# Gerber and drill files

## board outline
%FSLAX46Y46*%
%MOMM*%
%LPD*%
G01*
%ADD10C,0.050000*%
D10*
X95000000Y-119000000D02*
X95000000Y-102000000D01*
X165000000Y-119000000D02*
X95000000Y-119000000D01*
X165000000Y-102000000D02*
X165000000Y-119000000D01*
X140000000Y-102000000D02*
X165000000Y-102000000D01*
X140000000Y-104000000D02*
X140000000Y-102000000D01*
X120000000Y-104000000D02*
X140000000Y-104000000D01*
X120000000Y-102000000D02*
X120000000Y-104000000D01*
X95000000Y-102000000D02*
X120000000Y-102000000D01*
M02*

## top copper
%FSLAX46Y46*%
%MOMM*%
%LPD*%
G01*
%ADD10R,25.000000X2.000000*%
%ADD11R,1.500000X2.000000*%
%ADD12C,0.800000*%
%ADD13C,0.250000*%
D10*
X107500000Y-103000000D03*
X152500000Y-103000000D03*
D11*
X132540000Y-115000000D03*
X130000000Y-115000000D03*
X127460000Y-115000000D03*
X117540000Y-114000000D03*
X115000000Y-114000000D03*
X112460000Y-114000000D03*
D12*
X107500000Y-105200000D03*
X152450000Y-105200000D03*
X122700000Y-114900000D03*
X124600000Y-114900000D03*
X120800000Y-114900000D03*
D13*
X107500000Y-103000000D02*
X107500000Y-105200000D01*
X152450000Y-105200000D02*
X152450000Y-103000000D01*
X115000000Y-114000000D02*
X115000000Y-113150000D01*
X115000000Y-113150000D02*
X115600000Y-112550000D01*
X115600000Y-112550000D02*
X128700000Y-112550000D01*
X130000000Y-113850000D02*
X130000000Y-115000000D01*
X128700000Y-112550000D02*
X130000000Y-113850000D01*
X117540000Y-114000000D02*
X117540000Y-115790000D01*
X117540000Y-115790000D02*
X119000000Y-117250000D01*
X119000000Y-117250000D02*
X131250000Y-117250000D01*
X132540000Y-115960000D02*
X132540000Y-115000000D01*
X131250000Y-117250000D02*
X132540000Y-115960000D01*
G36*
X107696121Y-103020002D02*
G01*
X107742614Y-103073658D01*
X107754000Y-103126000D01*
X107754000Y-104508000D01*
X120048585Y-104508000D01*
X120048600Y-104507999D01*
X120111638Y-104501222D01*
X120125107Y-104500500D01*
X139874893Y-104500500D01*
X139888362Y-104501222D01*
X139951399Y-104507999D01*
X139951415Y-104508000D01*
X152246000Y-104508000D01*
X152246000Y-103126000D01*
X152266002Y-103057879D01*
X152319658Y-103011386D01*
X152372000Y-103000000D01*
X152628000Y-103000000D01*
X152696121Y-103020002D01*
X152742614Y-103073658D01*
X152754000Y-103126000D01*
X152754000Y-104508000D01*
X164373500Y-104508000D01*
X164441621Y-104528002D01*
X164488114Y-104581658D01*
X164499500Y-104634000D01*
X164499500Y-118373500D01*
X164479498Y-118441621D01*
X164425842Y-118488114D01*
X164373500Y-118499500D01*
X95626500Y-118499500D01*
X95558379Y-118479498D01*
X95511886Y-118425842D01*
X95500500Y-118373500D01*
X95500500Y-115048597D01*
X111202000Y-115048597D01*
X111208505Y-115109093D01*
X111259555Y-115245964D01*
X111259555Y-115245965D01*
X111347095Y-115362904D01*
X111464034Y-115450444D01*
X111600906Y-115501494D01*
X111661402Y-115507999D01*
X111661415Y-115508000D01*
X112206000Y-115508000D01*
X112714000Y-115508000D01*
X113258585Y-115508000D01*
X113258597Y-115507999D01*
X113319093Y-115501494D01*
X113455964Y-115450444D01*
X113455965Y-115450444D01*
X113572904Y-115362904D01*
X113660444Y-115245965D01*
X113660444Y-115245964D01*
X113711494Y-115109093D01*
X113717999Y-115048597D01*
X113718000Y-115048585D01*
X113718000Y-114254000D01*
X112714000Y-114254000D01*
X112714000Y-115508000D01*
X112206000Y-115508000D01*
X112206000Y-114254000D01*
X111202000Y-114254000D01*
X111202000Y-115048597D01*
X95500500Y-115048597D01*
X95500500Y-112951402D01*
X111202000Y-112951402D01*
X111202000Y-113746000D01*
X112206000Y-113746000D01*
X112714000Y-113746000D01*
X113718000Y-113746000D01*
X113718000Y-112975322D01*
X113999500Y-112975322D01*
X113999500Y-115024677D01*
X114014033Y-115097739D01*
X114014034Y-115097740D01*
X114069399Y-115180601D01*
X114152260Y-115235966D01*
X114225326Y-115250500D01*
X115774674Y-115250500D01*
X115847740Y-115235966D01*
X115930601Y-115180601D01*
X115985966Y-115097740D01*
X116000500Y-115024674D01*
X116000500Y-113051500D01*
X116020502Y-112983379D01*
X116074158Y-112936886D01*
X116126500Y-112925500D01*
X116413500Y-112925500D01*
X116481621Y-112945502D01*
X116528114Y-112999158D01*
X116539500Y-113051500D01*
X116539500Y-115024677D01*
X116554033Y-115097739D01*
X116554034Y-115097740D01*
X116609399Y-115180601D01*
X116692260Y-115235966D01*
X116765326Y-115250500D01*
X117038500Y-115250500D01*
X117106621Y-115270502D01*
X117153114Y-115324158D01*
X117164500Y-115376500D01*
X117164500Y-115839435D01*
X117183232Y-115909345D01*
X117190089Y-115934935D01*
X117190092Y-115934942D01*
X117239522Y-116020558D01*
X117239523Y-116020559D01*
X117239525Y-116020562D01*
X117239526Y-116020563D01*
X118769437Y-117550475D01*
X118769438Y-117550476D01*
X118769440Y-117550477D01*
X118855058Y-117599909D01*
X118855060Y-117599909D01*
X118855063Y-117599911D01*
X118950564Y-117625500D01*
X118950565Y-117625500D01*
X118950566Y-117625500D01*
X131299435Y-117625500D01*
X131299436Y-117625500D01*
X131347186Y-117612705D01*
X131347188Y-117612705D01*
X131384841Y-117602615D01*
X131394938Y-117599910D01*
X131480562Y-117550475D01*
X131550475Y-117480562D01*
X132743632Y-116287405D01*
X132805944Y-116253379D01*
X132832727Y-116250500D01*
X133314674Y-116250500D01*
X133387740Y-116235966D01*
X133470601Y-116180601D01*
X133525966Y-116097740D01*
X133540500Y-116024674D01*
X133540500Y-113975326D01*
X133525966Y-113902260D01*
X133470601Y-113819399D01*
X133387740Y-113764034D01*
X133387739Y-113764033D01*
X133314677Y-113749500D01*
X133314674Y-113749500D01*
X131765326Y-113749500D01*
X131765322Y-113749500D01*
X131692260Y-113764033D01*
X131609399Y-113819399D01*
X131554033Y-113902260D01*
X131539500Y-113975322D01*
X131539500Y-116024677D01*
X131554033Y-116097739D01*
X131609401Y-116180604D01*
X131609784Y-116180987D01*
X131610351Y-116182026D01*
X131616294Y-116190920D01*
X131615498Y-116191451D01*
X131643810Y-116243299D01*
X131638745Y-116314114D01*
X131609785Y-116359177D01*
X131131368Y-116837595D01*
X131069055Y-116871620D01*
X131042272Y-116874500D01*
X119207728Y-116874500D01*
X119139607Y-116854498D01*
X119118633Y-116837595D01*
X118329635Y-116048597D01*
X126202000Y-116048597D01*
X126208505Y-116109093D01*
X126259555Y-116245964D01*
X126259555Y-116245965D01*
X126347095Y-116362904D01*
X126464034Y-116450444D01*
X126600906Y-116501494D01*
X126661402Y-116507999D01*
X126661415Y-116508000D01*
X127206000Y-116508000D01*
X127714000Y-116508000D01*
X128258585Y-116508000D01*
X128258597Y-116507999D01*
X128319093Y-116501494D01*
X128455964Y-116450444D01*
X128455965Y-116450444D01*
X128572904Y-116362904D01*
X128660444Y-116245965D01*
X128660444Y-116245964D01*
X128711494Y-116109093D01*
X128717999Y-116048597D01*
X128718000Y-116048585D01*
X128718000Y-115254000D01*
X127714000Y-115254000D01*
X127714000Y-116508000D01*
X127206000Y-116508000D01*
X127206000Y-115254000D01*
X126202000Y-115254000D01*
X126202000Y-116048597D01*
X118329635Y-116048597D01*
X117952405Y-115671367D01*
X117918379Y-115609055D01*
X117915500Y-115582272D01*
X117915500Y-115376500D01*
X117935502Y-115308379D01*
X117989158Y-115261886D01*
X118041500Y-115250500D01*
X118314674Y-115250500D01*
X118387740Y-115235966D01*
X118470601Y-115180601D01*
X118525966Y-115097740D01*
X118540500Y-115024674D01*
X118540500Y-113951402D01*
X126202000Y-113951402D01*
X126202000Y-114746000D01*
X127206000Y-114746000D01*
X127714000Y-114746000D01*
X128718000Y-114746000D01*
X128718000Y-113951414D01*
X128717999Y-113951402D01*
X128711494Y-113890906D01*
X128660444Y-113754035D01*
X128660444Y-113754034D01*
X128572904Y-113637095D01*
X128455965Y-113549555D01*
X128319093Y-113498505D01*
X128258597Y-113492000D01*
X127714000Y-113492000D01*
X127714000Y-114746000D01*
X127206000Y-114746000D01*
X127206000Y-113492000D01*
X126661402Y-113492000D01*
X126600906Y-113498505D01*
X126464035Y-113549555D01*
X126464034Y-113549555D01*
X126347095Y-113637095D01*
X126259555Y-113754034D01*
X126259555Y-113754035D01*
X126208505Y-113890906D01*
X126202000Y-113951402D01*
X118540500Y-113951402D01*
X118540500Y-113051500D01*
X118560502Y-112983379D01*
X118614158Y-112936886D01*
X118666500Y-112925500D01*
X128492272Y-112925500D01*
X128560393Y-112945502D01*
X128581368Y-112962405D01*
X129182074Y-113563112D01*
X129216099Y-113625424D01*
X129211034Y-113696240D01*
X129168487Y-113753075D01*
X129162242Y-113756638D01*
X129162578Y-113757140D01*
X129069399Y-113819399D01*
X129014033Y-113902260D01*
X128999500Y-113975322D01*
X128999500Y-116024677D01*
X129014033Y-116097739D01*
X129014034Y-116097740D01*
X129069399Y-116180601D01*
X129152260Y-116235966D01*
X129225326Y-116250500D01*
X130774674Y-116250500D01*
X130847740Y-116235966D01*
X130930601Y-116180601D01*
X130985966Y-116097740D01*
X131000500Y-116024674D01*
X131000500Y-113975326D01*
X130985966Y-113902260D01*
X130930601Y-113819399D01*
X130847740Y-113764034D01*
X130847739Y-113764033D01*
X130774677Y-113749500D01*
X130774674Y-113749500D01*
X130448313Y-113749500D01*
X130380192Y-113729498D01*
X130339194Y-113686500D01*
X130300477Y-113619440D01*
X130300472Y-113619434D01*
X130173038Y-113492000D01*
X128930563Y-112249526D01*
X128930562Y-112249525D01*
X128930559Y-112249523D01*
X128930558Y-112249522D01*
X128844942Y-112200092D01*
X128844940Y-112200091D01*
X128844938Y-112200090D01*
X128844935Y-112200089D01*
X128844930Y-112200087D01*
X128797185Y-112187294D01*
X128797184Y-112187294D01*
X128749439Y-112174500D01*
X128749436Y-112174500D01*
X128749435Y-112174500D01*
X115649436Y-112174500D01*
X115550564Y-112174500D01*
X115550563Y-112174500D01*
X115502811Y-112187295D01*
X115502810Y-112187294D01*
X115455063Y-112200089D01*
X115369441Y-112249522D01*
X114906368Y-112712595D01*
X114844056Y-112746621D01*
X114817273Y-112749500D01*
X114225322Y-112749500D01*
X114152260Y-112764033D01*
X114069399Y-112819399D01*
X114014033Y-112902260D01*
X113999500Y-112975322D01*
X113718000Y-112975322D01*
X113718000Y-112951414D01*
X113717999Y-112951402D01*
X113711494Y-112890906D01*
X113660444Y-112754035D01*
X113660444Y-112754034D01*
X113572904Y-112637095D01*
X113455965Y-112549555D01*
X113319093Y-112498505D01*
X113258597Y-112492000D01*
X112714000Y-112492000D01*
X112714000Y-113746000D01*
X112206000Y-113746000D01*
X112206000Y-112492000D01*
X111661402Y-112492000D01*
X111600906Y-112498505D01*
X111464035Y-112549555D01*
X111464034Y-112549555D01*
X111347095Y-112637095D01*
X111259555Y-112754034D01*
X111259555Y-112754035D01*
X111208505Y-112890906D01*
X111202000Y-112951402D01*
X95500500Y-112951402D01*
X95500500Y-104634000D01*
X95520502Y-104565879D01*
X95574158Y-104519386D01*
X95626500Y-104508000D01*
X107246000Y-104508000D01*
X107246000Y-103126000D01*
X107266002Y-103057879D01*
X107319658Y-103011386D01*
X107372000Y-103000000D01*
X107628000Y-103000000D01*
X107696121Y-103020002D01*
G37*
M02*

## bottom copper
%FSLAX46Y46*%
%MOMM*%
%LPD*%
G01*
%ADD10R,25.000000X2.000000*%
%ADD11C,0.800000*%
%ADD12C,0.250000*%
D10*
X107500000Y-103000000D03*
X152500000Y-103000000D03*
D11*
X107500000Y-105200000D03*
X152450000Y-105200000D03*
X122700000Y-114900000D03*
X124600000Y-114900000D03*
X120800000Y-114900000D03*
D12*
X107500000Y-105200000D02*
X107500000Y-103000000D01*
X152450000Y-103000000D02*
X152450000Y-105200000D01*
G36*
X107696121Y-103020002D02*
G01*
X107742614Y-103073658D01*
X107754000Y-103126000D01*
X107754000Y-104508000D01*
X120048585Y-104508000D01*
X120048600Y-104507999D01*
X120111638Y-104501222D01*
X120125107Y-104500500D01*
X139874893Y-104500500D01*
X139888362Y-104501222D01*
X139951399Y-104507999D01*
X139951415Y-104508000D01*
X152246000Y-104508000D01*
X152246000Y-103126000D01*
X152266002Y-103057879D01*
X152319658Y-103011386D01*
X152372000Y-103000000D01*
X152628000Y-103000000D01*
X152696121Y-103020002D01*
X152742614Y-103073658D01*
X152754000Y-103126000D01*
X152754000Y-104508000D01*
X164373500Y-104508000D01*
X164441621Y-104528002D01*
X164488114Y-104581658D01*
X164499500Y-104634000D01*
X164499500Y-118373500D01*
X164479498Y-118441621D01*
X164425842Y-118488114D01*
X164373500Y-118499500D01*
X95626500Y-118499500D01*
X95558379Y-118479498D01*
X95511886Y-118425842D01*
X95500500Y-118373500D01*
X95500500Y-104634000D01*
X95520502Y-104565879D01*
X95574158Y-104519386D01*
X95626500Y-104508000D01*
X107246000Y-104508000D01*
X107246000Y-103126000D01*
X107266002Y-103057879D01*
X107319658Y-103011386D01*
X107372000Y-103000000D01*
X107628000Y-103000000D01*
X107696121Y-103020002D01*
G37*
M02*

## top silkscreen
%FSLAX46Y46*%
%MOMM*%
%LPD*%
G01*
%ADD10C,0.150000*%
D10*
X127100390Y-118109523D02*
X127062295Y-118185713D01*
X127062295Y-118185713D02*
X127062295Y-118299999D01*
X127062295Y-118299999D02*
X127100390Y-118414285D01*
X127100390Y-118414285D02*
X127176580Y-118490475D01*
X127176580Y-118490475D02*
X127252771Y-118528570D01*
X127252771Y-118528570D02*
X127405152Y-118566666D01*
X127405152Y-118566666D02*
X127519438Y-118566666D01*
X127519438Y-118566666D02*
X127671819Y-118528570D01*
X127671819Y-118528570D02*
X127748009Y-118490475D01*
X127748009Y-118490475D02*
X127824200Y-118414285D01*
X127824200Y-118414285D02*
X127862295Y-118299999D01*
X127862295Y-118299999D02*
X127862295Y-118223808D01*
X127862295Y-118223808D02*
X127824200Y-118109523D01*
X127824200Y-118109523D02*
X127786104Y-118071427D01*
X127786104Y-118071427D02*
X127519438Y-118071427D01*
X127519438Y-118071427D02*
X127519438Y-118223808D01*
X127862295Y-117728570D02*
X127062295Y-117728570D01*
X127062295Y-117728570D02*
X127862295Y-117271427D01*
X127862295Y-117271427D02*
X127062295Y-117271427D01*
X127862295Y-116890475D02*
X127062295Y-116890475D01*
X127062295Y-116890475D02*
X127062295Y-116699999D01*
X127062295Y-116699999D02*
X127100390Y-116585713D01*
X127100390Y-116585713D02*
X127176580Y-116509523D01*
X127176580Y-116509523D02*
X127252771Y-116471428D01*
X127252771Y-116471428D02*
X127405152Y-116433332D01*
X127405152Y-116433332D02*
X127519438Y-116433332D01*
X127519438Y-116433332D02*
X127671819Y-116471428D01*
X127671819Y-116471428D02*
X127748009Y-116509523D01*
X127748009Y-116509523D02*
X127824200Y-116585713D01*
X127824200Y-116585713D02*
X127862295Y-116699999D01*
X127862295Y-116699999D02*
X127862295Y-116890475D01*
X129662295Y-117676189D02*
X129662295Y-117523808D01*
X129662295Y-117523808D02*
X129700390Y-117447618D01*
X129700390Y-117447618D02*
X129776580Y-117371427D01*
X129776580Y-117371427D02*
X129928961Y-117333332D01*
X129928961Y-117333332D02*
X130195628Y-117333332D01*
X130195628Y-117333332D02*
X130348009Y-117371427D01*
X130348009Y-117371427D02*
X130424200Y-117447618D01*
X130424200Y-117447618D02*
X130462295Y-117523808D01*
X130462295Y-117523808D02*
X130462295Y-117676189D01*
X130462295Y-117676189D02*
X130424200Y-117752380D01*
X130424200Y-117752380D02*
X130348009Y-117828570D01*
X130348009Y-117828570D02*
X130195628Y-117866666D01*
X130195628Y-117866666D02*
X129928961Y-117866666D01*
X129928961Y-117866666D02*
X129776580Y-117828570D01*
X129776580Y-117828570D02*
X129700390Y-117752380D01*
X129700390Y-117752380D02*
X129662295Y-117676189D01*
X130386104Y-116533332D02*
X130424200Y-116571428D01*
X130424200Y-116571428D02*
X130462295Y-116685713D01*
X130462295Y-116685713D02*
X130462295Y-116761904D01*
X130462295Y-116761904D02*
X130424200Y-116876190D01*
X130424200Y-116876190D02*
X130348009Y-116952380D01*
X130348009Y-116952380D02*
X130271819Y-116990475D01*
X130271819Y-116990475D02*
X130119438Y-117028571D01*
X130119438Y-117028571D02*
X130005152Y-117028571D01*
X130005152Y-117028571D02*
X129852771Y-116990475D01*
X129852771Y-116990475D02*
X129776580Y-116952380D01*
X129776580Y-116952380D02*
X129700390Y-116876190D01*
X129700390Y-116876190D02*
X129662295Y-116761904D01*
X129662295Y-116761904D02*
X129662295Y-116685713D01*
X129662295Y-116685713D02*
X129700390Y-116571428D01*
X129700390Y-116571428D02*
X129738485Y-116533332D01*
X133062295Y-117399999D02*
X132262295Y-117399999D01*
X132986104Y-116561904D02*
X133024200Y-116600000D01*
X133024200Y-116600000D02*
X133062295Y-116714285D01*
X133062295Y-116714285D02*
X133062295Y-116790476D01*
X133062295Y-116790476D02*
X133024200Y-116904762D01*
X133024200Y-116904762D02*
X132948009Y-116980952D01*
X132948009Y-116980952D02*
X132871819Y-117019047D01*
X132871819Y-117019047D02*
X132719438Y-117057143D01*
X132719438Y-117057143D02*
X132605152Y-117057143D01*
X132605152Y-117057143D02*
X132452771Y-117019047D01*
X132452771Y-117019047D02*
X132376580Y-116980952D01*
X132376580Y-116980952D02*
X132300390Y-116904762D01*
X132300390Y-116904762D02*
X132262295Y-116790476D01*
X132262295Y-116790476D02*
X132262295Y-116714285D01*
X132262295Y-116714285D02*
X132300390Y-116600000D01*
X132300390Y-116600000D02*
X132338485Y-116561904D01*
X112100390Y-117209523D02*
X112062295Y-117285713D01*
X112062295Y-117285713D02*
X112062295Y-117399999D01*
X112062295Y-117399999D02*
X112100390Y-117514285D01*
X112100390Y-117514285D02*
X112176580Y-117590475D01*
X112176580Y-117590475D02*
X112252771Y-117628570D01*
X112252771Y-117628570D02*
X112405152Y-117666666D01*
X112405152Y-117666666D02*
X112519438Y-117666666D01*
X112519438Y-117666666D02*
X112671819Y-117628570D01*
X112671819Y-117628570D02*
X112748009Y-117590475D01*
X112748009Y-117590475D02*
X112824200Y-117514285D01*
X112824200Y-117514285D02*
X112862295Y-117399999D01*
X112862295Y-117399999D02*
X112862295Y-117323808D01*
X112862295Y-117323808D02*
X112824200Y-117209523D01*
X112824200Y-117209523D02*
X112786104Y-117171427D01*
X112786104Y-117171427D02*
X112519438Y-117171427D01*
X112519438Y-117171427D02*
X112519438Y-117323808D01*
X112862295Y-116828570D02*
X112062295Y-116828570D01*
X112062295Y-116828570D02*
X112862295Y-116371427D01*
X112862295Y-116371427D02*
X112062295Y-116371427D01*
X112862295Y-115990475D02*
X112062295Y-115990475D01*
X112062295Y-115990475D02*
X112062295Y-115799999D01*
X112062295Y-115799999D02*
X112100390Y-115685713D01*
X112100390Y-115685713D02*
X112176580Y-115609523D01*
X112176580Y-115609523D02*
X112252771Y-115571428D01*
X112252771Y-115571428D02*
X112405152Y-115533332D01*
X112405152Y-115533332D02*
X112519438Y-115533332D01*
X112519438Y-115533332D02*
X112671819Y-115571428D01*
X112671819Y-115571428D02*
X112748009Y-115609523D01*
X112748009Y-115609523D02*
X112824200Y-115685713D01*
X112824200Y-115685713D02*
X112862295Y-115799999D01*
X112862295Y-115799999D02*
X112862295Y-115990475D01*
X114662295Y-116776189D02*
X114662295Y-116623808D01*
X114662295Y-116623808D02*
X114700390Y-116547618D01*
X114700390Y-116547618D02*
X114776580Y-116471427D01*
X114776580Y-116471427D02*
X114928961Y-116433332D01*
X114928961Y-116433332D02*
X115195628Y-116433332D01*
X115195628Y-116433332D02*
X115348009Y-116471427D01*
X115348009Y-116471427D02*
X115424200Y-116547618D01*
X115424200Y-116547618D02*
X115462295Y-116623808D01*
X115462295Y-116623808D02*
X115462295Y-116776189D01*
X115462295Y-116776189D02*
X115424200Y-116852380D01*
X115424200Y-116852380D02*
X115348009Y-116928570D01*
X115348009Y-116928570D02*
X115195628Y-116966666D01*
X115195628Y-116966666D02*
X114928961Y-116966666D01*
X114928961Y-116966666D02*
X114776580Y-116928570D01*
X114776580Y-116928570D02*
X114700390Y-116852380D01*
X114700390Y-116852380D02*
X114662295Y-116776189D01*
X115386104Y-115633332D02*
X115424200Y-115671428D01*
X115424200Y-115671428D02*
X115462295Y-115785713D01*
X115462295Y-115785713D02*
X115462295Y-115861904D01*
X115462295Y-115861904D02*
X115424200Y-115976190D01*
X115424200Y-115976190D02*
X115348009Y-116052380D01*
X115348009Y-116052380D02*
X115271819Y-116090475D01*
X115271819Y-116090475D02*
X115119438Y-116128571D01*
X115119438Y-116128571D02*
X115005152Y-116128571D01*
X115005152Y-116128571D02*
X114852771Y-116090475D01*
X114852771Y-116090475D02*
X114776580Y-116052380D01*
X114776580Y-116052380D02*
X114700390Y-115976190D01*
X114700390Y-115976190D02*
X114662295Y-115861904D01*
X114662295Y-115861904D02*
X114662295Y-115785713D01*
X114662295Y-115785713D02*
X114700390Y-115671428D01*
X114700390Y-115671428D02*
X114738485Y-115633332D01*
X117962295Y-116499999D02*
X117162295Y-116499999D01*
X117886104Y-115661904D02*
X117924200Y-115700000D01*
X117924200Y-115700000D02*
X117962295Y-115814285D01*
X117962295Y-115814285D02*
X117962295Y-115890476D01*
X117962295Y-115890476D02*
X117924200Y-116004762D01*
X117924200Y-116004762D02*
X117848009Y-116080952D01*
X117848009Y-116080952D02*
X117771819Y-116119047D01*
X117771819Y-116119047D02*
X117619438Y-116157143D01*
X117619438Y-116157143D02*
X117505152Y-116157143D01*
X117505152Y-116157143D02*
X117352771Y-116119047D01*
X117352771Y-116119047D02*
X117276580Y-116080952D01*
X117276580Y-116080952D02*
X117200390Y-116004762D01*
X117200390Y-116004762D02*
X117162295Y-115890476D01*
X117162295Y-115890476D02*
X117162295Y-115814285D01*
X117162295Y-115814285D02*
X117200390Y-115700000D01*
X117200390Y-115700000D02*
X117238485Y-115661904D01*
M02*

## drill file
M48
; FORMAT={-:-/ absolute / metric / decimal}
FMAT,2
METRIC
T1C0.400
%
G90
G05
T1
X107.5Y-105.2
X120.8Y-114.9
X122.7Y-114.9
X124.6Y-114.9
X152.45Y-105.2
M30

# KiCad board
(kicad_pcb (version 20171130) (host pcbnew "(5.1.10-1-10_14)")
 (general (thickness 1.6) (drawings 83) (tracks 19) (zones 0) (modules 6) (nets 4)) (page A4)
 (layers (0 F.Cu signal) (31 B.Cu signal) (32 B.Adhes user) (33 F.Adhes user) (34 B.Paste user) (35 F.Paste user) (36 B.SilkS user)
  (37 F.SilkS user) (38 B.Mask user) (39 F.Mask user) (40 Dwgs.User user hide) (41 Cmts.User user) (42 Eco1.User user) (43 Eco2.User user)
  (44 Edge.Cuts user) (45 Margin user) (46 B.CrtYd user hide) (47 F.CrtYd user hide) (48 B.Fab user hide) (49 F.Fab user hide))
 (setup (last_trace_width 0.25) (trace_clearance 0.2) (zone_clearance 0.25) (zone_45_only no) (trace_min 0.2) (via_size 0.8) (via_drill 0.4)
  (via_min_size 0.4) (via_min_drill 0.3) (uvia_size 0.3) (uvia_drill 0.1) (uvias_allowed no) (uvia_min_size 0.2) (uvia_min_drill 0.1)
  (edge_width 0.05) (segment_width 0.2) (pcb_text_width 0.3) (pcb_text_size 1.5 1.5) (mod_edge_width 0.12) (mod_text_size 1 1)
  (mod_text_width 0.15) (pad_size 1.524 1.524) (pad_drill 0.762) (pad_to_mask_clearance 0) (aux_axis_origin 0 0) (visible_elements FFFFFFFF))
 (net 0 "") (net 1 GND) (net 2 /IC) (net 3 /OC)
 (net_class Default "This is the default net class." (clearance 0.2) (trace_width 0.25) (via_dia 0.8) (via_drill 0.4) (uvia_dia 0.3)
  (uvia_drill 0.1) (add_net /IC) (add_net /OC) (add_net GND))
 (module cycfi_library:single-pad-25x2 (layer F.Cu) (at 107.5 103)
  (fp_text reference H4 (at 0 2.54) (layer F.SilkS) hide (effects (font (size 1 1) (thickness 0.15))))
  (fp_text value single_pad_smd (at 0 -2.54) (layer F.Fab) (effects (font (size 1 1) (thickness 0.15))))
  (pad 1 smd rect (at 0 0) (size 25 2) (layers F.Cu F.Paste F.Mask) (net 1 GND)))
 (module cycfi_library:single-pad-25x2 (layer B.Cu) (at 107.5 103)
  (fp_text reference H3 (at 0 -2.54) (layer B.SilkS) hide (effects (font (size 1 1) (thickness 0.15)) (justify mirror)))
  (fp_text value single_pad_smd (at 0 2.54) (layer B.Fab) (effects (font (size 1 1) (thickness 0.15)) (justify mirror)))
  (pad 1 smd rect (at 0 0) (size 25 2) (layers B.Cu B.Paste B.Mask) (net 1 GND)))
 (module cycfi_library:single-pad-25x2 (layer F.Cu) (at 152.5 103)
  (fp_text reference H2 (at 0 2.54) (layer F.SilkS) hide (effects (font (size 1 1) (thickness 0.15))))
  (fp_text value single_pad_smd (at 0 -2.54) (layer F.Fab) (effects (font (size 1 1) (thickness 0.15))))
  (pad 1 smd rect (at 0 0) (size 25 2) (layers F.Cu F.Paste F.Mask) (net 1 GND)))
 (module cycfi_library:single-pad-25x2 (layer B.Cu) (at 152.5 103)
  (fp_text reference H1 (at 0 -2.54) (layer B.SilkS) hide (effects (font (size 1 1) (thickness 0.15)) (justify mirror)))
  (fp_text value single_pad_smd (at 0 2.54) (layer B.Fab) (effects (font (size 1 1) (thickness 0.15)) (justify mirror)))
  (pad 1 smd rect (at 0 0) (size 25 2) (layers B.Cu B.Paste B.Mask) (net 1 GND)))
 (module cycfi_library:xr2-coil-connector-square (layer F.Cu) (at 130 115)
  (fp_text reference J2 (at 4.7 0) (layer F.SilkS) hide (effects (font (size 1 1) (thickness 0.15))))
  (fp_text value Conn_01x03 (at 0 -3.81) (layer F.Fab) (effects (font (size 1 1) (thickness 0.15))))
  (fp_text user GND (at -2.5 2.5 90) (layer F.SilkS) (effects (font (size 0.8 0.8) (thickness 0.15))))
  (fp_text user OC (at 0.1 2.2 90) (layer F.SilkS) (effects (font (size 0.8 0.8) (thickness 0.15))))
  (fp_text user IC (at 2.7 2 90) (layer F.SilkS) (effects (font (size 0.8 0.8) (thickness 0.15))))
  (pad 3 smd rect (at 2.54 0) (size 1.5 2) (layers F.Cu F.Paste F.Mask) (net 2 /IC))
  (pad 2 smd rect (at 0 0) (size 1.5 2) (layers F.Cu F.Paste F.Mask) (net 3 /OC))
  (pad 1 smd rect (at -2.54 0) (size 1.5 2) (layers F.Cu F.Paste F.Mask) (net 1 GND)))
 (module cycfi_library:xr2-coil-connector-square (layer F.Cu) (at 115 114)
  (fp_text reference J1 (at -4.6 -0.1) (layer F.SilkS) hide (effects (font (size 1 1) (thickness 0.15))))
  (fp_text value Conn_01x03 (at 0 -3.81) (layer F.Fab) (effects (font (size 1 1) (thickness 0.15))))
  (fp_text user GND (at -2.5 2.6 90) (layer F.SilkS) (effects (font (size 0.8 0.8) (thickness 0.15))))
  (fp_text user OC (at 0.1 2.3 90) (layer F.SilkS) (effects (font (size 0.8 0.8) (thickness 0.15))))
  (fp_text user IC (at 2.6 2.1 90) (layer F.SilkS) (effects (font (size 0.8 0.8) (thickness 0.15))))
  (pad 3 smd rect (at 2.54 0) (size 1.5 2) (layers F.Cu F.Paste F.Mask) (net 2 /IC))
  (pad 2 smd rect (at 0 0) (size 1.5 2) (layers F.Cu F.Paste F.Mask) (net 3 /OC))
  (pad 1 smd rect (at -2.54 0) (size 1.5 2) (layers F.Cu F.Paste F.Mask) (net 1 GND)))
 (gr_line (start 95 119) (end 95 102) (layer Edge.Cuts) (width 0.05))
 (gr_line (start 165 119) (end 95 119) (layer Edge.Cuts) (width 0.05))
 (gr_line (start 165 102) (end 165 119) (layer Edge.Cuts) (width 0.05))
 (gr_line (start 140 102) (end 165 102) (layer Edge.Cuts) (width 0.05))
 (gr_line (start 140 104) (end 140 102) (layer Edge.Cuts) (width 0.05))
 (gr_line (start 120 104) (end 140 104) (layer Edge.Cuts) (width 0.05))
 (gr_line (start 120 102) (end 120 104) (layer Edge.Cuts) (width 0.05))
 (gr_line (start 95 102) (end 120 102) (layer Edge.Cuts) (width 0.05))
 (via (at 107.5 105.2) (size 0.8) (drill 0.4) (layers F.Cu B.Cu) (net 1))
 (segment (start 107.5 103) (end 107.5 105.2) (width 0.25) (layer F.Cu) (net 1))
 (segment (start 107.5 105.2) (end 107.5 103) (width 0.25) (layer B.Cu) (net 1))
 (via (at 152.45 105.2) (size 0.8) (drill 0.4) (layers F.Cu B.Cu) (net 1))
 (segment (start 152.45 103) (end 152.45 105.2) (width 0.25) (layer B.Cu) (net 1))
 (segment (start 152.45 105.2) (end 152.45 103) (width 0.25) (layer F.Cu) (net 1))
 (via (at 122.7 114.9) (size 0.8) (drill 0.4) (layers F.Cu B.Cu) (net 1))
 (via (at 124.6 114.9) (size 0.8) (drill 0.4) (layers F.Cu B.Cu) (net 1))
 (via (at 120.8 114.9) (size 0.8) (drill 0.4) (layers F.Cu B.Cu) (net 1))
 (segment (start 115 114) (end 115 113.15) (width 0.25) (layer F.Cu) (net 3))
 (segment (start 115 113.15) (end 115.6 112.55) (width 0.25) (layer F.Cu) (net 3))
 (segment (start 115.6 112.55) (end 128.7 112.55) (width 0.25) (layer F.Cu) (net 3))
 (segment (start 130 113.85) (end 130 115) (width 0.25) (layer F.Cu) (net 3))
 (segment (start 128.7 112.55) (end 130 113.85) (width 0.25) (layer F.Cu) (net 3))
 (segment (start 117.54 114) (end 117.54 115.79) (width 0.25) (layer F.Cu) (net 2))
 (segment (start 117.54 115.79) (end 119 117.25) (width 0.25) (layer F.Cu) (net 2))
 (segment (start 119 117.25) (end 131.25 117.25) (width 0.25) (layer F.Cu) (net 2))
 (segment (start 132.54 115.96) (end 132.54 115) (width 0.25) (layer F.Cu) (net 2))
 (segment (start 131.25 117.25) (end 132.54 115.96) (width 0.25) (layer F.Cu) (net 2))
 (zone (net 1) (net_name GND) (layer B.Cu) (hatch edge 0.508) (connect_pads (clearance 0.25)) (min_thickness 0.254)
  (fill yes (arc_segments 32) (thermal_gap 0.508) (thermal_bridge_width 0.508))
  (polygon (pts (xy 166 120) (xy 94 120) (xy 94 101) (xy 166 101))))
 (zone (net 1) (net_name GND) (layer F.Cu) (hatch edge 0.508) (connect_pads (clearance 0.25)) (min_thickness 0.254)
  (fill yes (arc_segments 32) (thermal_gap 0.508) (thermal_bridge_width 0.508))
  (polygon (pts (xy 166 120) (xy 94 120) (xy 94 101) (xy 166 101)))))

